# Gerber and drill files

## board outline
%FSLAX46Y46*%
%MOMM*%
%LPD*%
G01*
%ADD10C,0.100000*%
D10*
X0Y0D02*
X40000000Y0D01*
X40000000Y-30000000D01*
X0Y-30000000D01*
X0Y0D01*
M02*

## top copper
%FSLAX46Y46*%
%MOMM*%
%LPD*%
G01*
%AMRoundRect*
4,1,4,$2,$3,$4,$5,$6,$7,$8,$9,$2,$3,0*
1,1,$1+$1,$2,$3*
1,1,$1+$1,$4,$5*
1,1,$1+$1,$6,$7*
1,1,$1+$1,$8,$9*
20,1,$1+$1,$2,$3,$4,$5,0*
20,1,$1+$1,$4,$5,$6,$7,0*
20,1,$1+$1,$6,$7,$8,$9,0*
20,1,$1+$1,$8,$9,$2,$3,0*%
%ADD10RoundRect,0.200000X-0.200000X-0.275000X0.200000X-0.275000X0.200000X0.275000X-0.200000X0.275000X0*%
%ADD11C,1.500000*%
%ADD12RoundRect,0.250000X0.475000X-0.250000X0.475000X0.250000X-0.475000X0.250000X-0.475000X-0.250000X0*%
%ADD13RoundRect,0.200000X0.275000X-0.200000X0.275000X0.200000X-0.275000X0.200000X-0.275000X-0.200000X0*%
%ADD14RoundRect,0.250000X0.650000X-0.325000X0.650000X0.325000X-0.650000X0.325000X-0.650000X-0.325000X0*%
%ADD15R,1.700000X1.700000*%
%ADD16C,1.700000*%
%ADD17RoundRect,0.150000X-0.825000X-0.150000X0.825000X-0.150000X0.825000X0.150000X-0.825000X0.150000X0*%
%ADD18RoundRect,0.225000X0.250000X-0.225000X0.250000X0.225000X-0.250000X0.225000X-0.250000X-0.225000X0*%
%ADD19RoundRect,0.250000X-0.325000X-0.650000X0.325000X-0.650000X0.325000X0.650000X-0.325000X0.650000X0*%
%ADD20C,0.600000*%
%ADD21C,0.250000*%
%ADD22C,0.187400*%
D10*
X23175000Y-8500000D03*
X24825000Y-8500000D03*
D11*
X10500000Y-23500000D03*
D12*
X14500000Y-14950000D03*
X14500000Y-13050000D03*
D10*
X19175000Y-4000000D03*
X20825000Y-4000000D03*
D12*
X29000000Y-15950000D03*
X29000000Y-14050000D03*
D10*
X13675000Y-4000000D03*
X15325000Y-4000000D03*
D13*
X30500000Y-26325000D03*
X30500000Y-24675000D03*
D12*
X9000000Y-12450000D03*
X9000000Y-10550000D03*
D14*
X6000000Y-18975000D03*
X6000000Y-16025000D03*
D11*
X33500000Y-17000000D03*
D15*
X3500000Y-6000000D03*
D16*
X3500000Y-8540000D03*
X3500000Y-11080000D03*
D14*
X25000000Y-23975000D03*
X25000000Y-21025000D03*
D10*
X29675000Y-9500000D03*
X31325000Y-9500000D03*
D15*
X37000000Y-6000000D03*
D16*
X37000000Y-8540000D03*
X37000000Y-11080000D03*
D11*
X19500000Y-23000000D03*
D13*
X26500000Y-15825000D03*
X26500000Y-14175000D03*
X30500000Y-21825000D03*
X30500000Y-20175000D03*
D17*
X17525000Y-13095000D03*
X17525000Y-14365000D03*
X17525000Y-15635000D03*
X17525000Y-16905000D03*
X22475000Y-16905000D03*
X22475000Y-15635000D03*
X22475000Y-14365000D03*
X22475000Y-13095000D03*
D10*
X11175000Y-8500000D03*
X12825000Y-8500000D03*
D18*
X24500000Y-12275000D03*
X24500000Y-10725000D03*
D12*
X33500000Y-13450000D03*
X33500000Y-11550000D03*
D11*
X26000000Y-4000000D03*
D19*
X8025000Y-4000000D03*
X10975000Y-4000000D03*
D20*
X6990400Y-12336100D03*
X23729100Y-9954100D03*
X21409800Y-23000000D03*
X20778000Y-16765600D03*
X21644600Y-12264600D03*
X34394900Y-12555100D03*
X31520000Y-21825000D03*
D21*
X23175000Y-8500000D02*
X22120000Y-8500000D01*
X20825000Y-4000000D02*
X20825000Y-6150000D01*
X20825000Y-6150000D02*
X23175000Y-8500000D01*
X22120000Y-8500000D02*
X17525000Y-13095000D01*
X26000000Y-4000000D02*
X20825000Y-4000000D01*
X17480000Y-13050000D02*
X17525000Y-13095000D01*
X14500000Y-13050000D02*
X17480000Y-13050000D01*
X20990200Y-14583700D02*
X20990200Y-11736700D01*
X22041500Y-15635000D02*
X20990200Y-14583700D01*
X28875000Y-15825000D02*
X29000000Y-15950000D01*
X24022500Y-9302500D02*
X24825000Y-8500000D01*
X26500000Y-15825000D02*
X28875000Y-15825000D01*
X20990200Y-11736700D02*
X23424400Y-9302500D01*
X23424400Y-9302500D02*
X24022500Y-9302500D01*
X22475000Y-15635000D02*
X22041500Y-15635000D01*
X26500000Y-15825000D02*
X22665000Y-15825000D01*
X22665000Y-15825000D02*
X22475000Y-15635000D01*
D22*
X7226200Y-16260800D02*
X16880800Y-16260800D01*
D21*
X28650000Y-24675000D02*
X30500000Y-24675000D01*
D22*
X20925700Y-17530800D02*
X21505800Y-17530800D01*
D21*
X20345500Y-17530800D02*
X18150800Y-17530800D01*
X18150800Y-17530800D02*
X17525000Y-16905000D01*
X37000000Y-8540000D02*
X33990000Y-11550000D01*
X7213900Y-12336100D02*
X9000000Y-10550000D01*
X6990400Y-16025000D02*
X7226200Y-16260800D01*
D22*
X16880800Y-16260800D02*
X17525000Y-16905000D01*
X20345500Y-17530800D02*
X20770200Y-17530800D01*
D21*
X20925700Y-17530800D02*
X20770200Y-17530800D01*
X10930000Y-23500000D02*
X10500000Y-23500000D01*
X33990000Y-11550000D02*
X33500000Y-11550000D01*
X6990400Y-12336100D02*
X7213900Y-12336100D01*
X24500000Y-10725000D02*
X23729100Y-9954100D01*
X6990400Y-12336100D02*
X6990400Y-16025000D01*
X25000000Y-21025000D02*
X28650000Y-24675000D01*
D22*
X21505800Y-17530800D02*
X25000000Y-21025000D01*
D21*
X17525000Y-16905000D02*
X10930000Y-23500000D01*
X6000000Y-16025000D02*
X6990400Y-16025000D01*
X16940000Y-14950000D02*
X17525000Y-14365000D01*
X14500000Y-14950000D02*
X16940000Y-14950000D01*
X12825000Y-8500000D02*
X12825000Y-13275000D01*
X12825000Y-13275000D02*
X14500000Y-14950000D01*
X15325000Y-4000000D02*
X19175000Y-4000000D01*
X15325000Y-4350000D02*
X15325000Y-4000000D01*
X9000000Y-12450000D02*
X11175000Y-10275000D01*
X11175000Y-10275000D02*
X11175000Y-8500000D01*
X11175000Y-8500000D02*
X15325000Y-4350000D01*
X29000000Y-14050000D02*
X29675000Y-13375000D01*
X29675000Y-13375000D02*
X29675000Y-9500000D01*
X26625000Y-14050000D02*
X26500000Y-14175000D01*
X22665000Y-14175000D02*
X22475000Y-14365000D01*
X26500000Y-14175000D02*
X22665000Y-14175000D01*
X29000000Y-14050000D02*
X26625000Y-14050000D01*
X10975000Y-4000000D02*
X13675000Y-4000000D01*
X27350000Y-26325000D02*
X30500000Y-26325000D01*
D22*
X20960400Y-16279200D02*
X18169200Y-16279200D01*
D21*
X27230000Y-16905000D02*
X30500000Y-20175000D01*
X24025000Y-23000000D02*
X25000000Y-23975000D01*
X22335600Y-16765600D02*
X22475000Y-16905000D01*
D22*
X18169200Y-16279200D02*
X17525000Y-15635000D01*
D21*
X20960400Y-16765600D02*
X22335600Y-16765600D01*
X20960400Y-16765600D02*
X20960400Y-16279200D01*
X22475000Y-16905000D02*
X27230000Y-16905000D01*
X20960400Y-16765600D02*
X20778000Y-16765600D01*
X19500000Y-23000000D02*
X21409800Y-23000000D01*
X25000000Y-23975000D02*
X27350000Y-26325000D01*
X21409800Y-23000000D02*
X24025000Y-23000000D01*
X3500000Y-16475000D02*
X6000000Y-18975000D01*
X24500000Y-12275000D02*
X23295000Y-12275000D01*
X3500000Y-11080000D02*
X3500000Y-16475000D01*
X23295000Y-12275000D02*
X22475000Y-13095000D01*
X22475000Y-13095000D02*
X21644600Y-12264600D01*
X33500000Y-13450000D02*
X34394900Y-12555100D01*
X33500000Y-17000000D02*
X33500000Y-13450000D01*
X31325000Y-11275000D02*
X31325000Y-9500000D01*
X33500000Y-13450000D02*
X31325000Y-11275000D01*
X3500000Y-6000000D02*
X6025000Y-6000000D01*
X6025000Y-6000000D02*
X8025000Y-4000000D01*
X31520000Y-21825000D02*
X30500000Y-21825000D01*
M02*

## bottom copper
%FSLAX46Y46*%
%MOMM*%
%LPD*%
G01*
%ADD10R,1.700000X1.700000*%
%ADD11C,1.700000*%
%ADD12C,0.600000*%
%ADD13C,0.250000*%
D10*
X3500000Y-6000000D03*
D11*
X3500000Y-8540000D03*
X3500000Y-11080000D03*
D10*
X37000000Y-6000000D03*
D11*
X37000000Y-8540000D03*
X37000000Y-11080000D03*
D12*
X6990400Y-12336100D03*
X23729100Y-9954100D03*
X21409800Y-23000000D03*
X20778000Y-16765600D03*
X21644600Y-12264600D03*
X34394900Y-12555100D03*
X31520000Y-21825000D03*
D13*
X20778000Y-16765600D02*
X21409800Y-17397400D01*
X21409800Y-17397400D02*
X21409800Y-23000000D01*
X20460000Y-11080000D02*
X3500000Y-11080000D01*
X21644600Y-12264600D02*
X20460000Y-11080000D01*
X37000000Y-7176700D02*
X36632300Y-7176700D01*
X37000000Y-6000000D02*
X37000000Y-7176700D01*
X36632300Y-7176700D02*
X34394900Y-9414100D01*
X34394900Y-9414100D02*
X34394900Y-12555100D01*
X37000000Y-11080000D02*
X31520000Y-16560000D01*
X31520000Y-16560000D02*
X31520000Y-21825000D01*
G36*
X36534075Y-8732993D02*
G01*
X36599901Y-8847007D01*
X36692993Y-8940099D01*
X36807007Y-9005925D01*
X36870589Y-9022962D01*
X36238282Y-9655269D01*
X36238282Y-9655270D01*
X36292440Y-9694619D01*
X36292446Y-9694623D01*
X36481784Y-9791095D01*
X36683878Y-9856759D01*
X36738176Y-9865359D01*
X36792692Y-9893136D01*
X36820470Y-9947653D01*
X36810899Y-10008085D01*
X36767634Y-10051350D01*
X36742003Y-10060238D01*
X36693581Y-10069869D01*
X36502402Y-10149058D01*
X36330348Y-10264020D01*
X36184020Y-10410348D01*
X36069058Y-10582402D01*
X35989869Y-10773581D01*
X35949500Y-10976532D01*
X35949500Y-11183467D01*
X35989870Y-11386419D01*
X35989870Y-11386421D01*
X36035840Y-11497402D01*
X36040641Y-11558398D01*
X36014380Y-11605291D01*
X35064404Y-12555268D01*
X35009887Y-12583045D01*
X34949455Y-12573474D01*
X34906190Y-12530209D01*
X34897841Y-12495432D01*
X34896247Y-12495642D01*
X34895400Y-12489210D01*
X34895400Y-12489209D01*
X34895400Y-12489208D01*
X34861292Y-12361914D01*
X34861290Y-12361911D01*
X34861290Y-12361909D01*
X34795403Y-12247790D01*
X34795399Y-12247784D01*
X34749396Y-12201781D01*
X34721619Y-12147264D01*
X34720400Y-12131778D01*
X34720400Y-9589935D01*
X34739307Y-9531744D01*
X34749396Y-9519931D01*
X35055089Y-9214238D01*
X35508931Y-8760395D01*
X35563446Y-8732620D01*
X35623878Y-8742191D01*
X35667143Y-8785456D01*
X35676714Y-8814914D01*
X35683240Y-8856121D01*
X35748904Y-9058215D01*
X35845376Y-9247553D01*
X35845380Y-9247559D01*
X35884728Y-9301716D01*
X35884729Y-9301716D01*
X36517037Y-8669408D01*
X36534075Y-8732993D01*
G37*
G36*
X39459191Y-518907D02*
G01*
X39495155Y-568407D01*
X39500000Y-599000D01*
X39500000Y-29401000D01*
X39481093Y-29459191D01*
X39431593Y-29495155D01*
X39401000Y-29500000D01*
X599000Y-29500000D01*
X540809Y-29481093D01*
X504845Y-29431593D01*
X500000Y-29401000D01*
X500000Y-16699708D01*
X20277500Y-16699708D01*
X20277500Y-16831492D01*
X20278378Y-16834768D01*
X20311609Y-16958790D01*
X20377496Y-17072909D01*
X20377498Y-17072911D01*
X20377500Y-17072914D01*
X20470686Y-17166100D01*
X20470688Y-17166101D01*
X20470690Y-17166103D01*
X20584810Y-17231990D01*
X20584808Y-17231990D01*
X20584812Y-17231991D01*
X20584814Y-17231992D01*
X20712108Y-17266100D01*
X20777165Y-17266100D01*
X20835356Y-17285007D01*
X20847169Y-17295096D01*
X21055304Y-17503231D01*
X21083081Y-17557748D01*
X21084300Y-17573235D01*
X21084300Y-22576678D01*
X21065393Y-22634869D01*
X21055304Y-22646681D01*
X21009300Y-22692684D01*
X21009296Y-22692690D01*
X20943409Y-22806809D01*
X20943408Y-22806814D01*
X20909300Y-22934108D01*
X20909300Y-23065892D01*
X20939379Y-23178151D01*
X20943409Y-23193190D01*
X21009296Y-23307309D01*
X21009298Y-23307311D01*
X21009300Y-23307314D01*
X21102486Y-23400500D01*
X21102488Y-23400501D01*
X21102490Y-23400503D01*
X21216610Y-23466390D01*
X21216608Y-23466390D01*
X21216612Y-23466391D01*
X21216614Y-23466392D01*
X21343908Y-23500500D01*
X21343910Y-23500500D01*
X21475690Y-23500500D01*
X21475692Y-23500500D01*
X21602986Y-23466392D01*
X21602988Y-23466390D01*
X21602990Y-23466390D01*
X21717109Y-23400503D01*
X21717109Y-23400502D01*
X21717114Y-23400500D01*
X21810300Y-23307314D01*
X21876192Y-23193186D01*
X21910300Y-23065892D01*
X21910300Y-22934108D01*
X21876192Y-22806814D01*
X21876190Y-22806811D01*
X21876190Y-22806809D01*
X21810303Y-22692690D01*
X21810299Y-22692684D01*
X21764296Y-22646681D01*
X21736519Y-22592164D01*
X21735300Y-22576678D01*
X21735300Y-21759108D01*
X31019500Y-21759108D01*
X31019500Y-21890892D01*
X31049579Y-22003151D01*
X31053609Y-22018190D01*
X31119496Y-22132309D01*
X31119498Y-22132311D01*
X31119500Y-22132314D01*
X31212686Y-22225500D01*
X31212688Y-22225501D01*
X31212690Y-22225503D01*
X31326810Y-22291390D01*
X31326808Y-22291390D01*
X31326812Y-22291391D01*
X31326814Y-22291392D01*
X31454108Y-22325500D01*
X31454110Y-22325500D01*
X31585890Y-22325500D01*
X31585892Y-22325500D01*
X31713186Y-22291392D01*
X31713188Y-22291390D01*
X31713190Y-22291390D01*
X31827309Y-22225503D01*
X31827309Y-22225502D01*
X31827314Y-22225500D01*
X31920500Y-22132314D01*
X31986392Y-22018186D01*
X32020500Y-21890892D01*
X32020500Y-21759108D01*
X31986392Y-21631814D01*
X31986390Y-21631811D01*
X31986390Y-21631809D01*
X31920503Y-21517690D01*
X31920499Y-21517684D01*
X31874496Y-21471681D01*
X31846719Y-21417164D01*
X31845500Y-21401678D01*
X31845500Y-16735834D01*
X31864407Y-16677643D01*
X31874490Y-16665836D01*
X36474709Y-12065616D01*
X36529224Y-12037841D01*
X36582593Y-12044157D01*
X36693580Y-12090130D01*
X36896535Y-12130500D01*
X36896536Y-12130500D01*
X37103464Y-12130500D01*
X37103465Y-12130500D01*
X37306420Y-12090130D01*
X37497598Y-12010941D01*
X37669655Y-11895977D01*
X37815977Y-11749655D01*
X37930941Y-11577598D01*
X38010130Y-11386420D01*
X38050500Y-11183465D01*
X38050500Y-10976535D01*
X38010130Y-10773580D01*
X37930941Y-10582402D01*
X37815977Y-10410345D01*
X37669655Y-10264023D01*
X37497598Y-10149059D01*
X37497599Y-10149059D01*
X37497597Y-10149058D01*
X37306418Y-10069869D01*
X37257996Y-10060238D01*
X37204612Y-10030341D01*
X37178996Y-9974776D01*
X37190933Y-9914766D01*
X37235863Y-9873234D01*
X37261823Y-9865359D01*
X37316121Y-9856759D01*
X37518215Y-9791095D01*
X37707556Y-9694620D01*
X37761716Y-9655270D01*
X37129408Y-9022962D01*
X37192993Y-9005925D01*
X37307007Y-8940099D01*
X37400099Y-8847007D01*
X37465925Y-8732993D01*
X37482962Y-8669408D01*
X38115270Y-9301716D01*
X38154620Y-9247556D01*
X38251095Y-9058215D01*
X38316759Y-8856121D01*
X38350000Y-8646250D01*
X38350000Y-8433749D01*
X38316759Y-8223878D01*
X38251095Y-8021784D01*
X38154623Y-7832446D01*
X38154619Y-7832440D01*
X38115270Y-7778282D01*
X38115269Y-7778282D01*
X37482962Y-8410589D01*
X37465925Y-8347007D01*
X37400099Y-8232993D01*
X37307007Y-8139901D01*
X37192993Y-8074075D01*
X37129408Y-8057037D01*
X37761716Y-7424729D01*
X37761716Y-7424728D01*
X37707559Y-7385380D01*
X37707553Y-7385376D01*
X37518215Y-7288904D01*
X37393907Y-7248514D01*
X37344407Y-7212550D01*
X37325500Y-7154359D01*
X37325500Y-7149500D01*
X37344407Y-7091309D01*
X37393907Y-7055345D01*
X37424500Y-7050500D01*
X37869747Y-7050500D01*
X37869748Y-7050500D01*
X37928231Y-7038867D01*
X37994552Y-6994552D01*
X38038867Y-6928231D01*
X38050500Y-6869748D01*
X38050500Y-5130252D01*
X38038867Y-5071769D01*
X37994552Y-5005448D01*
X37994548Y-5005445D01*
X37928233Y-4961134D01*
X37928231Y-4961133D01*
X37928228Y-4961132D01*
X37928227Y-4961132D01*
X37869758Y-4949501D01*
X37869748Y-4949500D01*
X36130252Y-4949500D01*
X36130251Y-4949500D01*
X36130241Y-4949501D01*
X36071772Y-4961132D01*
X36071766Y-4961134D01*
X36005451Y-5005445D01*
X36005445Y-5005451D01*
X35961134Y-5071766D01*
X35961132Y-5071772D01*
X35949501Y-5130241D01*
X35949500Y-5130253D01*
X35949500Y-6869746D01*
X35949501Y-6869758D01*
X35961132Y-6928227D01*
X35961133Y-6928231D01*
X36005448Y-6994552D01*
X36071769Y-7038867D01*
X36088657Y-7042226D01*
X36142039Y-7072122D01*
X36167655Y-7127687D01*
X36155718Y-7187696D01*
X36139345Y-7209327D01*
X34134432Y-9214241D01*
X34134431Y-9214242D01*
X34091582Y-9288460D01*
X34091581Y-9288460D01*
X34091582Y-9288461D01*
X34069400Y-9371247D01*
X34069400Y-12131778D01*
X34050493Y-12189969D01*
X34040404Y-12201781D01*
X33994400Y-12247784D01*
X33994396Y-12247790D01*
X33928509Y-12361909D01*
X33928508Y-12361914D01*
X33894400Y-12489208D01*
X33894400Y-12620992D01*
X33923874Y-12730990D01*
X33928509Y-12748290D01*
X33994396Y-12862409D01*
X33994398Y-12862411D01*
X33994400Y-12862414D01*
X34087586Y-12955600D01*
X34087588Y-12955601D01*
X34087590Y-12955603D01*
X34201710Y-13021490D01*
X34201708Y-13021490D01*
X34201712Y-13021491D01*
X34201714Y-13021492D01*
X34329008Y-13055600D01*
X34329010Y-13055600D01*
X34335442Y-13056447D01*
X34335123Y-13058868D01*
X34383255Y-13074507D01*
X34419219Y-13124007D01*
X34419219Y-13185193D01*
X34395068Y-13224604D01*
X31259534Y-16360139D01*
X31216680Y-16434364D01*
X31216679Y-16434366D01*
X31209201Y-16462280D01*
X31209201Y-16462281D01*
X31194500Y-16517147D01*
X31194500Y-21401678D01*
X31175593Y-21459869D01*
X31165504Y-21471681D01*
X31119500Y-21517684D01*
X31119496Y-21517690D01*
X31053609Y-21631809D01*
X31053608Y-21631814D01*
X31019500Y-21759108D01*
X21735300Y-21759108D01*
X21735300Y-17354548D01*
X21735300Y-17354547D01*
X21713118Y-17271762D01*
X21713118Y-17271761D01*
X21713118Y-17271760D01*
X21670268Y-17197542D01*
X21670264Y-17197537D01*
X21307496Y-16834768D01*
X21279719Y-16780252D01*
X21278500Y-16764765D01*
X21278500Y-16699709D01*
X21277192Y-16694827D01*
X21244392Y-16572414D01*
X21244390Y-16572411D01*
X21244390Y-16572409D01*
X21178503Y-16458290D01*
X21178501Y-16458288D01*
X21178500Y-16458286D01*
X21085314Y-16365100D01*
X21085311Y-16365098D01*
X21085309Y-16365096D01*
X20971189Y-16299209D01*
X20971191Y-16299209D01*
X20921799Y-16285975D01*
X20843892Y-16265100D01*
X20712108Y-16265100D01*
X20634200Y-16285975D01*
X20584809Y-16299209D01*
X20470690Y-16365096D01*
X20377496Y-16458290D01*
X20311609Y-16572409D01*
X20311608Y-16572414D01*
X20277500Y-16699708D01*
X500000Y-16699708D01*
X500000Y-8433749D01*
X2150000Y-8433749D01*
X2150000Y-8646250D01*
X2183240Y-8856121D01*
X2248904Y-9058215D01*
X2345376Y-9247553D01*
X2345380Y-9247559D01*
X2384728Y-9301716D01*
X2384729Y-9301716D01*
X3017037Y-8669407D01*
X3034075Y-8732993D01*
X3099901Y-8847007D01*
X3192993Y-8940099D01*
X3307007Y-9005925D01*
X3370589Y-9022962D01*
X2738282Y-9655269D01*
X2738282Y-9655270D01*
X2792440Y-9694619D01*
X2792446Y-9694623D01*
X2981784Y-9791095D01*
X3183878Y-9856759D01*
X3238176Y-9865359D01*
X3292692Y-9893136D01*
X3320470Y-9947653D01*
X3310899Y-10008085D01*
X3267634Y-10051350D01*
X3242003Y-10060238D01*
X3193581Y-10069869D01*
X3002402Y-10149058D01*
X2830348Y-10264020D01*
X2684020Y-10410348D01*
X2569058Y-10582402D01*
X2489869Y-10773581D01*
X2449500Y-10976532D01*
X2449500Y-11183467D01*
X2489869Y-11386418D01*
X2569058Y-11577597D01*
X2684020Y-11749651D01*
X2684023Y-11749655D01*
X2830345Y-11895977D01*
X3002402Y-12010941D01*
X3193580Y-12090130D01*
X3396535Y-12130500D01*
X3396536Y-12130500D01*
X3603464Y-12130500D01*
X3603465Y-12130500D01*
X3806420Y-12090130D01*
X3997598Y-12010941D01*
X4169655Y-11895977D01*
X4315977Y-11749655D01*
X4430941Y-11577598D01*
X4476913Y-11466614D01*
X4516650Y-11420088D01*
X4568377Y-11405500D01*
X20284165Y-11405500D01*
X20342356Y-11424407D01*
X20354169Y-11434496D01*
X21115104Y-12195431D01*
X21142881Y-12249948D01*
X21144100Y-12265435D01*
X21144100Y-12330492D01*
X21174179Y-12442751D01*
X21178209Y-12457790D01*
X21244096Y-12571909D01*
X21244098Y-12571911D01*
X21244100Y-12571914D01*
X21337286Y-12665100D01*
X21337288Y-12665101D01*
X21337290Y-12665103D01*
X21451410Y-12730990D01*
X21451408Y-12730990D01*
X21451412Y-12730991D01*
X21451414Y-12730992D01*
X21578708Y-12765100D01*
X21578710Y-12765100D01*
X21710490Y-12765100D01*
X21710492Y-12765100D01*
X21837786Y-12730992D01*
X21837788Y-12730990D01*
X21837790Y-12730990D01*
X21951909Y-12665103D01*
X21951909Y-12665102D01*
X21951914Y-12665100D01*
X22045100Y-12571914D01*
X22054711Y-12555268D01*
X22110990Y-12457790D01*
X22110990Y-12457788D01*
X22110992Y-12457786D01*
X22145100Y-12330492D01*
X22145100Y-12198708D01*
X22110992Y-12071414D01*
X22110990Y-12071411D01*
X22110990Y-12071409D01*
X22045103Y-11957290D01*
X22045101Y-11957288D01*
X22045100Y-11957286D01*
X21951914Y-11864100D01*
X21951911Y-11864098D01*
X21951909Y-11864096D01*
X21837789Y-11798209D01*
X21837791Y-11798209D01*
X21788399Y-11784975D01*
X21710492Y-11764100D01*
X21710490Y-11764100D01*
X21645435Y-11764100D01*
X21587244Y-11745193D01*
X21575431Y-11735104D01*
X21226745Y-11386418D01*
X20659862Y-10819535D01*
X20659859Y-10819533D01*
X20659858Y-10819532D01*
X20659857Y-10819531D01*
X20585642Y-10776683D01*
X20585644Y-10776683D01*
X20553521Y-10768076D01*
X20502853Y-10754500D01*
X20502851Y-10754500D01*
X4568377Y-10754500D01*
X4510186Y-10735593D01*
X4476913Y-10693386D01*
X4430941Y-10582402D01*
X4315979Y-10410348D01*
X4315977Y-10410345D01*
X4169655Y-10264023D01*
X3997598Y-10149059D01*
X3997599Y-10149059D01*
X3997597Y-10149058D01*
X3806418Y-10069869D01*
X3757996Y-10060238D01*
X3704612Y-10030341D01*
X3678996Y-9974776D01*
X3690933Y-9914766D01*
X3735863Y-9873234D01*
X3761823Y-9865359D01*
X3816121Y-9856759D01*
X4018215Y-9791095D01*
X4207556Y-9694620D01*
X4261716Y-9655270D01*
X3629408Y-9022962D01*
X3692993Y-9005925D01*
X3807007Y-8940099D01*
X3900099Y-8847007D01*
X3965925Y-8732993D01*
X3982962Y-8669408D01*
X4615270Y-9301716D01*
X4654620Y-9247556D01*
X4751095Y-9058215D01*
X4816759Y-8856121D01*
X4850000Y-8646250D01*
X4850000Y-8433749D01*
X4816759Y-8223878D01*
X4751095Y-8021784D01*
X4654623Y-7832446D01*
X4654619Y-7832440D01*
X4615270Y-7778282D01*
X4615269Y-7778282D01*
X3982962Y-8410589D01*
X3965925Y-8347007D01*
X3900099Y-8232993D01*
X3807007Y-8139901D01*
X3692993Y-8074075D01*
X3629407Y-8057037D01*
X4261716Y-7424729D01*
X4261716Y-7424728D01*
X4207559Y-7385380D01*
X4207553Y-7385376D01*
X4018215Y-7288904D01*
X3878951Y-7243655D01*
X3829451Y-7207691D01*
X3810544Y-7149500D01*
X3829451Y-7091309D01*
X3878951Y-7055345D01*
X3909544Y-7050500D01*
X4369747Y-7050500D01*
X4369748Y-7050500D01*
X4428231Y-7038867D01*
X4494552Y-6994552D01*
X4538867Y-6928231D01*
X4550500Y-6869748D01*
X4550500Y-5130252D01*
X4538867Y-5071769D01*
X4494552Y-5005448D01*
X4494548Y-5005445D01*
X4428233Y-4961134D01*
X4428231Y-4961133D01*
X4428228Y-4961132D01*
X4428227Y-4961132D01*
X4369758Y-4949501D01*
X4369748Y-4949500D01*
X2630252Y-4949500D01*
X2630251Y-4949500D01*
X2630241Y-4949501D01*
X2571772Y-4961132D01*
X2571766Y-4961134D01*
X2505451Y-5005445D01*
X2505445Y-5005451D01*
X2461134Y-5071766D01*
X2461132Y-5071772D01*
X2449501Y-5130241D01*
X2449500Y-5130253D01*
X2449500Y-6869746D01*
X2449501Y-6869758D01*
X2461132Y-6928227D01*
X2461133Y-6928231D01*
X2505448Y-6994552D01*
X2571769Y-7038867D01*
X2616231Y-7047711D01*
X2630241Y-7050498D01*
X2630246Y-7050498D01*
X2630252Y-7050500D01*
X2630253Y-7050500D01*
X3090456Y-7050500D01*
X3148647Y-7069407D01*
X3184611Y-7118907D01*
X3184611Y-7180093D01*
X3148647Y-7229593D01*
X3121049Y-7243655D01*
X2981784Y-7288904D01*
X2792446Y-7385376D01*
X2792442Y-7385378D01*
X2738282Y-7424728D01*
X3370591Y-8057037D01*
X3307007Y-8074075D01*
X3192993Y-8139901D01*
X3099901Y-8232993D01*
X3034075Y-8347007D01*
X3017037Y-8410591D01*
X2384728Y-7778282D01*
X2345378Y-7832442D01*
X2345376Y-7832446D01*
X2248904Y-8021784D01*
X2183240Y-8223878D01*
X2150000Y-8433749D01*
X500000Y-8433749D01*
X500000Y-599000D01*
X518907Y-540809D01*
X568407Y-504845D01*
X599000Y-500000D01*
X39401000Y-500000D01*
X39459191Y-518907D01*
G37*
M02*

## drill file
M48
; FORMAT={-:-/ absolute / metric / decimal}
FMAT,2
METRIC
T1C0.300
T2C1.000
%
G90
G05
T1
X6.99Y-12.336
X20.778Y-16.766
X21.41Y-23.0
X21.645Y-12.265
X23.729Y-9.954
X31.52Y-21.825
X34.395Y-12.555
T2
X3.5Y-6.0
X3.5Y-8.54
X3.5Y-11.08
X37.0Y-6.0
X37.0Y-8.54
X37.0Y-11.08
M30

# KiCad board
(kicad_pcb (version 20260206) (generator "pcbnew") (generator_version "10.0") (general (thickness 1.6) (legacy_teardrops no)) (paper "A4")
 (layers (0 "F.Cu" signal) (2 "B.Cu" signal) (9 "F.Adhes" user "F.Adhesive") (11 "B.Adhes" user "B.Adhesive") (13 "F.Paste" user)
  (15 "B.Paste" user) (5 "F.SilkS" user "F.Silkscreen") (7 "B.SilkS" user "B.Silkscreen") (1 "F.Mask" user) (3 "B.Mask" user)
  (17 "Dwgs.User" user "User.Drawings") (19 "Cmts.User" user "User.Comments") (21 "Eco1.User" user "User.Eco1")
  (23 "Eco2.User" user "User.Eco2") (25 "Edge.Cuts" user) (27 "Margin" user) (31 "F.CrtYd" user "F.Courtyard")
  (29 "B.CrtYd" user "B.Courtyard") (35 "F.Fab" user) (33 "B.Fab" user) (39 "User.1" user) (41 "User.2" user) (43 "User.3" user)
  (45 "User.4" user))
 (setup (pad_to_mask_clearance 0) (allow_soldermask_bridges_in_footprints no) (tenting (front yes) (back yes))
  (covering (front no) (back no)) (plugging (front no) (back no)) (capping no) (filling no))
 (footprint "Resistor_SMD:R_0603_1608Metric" (layer "F.Cu") (at 24 8.5)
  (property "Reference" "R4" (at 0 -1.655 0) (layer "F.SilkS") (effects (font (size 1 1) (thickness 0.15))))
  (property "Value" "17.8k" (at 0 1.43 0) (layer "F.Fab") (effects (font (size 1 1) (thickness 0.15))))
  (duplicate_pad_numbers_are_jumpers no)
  (pad "1" smd roundrect (at -0.825 0) (size 0.8 0.95) (layers "F.Cu" "F.Mask" "F.Paste") (roundrect_rratio 0.25) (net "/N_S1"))
  (pad "2" smd roundrect (at 0.825 0) (size 0.8 0.95) (layers "F.Cu" "F.Mask" "F.Paste") (roundrect_rratio 0.25) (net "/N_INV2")))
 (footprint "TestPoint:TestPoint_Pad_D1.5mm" (layer "F.Cu") (at 10.5 23.5)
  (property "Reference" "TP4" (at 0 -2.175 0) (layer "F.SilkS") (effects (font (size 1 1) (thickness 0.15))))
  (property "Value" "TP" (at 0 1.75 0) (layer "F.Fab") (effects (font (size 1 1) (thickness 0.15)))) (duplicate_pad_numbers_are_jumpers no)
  (pad "1" smd circle (at 0 0) (size 1.5 1.5) (layers "F.Cu" "F.Mask") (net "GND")))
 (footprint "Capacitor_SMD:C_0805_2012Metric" (layer "F.Cu") (at 14.5 14 90)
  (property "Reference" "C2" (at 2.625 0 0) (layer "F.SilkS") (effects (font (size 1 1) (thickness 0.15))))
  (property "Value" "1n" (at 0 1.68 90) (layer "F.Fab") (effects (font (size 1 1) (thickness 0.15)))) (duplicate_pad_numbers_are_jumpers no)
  (pad "1" smd roundrect (at -0.95 0 90) (size 1 1.45) (layers "F.Cu" "F.Mask" "F.Paste") (roundrect_rratio 0.25) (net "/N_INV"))
  (pad "2" smd roundrect (at 0.95 0 90) (size 1 1.45) (layers "F.Cu" "F.Mask" "F.Paste") (roundrect_rratio 0.25) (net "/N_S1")))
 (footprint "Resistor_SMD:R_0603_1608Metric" (layer "F.Cu") (at 20 4)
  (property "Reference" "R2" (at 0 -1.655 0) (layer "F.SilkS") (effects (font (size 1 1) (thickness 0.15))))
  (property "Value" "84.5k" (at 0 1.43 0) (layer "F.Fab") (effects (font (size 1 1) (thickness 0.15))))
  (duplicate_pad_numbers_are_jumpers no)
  (pad "1" smd roundrect (at -0.825 0) (size 0.8 0.95) (layers "F.Cu" "F.Mask" "F.Paste") (roundrect_rratio 0.25) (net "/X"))
  (pad "2" smd roundrect (at 0.825 0) (size 0.8 0.95) (layers "F.Cu" "F.Mask" "F.Paste") (roundrect_rratio 0.25) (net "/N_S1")))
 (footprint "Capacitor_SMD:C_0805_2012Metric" (layer "F.Cu") (at 29 15 90)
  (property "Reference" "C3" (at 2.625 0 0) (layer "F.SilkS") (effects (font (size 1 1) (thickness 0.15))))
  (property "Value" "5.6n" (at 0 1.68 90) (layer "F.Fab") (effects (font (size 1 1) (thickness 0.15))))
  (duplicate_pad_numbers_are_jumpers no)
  (pad "1" smd roundrect (at -0.95 0 90) (size 1 1.45) (layers "F.Cu" "F.Mask" "F.Paste") (roundrect_rratio 0.25) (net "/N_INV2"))
  (pad "2" smd roundrect (at 0.95 0 90) (size 1 1.45) (layers "F.Cu" "F.Mask" "F.Paste") (roundrect_rratio 0.25) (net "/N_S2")))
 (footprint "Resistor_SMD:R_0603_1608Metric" (layer "F.Cu") (at 14.5 4)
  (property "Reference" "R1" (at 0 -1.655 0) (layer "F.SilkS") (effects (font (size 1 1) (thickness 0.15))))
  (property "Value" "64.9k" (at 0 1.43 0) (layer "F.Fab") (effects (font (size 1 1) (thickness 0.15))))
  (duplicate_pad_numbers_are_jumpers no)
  (pad "1" smd roundrect (at -0.825 0) (size 0.8 0.95) (layers "F.Cu" "F.Mask" "F.Paste") (roundrect_rratio 0.25) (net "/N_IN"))
  (pad "2" smd roundrect (at 0.825 0) (size 0.8 0.95) (layers "F.Cu" "F.Mask" "F.Paste") (roundrect_rratio 0.25) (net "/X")))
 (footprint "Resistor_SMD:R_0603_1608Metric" (layer "F.Cu") (at 30.5 25.5 90)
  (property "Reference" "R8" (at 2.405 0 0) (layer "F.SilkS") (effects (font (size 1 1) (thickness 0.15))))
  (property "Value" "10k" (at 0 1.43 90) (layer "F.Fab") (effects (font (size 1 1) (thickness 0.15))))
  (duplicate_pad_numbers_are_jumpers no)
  (pad "1" smd roundrect (at -0.825 0 90) (size 0.8 0.95) (layers "F.Cu" "F.Mask" "F.Paste") (roundrect_rratio 0.25) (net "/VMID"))
  (pad "2" smd roundrect (at 0.825 0 90) (size 0.8 0.95) (layers "F.Cu" "F.Mask" "F.Paste") (roundrect_rratio 0.25) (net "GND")))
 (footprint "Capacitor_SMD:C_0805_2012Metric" (layer "F.Cu") (at 9 11.5 90)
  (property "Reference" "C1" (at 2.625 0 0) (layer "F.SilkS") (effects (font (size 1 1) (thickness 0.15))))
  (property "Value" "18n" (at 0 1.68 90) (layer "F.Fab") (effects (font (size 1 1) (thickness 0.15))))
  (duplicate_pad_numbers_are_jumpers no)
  (pad "1" smd roundrect (at -0.95 0 90) (size 1 1.45) (layers "F.Cu" "F.Mask" "F.Paste") (roundrect_rratio 0.25) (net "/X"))
  (pad "2" smd roundrect (at 0.95 0 90) (size 1 1.45) (layers "F.Cu" "F.Mask" "F.Paste") (roundrect_rratio 0.25) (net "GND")))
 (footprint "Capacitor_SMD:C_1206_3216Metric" (layer "F.Cu") (at 6 17.5 90)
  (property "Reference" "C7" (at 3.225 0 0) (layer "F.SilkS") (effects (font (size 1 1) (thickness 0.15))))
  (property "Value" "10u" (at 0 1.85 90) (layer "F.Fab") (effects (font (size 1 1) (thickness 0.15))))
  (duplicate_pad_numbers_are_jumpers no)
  (pad "1" smd roundrect (at -1.475 0 90) (size 1.15 1.8) (layers "F.Cu" "F.Mask" "F.Paste") (roundrect_rratio 0.217391) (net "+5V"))
  (pad "2" smd roundrect (at 1.475 0 90) (size 1.15 1.8) (layers "F.Cu" "F.Mask" "F.Paste") (roundrect_rratio 0.217391) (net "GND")))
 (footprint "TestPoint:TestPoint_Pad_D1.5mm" (layer "F.Cu") (at 33.5 17)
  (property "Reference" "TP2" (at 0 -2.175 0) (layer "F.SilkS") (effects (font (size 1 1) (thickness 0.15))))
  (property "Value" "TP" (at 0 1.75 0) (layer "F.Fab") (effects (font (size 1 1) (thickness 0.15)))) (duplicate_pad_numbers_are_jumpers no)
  (pad "1" smd circle (at 0 0) (size 1.5 1.5) (layers "F.Cu" "F.Mask") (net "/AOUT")))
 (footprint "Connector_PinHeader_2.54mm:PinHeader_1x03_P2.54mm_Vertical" (layer "F.Cu") (at 3.5 6)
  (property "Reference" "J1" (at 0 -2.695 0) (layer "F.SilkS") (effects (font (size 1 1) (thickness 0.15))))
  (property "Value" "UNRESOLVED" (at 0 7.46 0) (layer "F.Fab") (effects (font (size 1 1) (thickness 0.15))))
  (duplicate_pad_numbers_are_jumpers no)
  (pad "1" thru_hole rect (at 0 0) (size 1.7 1.7) (drill 1) (layers "*.Cu" "*.Mask") (remove_unused_layers no) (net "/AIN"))
  (pad "2" thru_hole circle (at 0 2.54) (size 1.7 1.7) (drill 1) (layers "*.Cu" "*.Mask") (remove_unused_layers no) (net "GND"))
  (pad "3" thru_hole circle (at 0 5.08) (size 1.7 1.7) (drill 1) (layers "*.Cu" "*.Mask") (remove_unused_layers no) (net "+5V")))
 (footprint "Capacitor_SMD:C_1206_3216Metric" (layer "F.Cu") (at 25 22.5 90)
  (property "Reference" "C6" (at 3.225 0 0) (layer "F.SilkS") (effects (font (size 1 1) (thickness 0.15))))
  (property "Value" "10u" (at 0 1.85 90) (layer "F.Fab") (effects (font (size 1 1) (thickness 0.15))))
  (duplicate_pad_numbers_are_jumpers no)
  (pad "1" smd roundrect (at -1.475 0 90) (size 1.15 1.8) (layers "F.Cu" "F.Mask" "F.Paste") (roundrect_rratio 0.217391) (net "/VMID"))
  (pad "2" smd roundrect (at 1.475 0 90) (size 1.15 1.8) (layers "F.Cu" "F.Mask" "F.Paste") (roundrect_rratio 0.217391) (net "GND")))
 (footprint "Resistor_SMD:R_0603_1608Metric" (layer "F.Cu") (at 30.5 9.5)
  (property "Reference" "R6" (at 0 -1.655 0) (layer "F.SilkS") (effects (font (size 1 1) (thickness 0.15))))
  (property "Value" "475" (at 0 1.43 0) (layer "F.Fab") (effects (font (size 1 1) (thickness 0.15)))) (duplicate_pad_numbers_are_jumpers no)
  (pad "1" smd roundrect (at -0.825 0) (size 0.8 0.95) (layers "F.Cu" "F.Mask" "F.Paste") (roundrect_rratio 0.25) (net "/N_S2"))
  (pad "2" smd roundrect (at 0.825 0) (size 0.8 0.95) (layers "F.Cu" "F.Mask" "F.Paste") (roundrect_rratio 0.25) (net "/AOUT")))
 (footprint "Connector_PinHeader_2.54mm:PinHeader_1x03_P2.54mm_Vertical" (layer "F.Cu") (at 37 6)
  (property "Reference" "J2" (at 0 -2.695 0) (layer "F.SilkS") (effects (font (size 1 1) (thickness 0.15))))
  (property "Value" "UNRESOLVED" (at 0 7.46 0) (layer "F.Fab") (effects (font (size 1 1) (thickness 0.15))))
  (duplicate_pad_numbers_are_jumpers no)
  (pad "1" thru_hole rect (at 0 0) (size 1.7 1.7) (drill 1) (layers "*.Cu" "*.Mask") (remove_unused_layers no) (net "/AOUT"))
  (pad "2" thru_hole circle (at 0 2.54) (size 1.7 1.7) (drill 1) (layers "*.Cu" "*.Mask") (remove_unused_layers no) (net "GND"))
  (pad "3" thru_hole circle (at 0 5.08) (size 1.7 1.7) (drill 1) (layers "*.Cu" "*.Mask") (remove_unused_layers no) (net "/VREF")))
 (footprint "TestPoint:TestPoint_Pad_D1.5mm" (layer "F.Cu") (at 19.5 23)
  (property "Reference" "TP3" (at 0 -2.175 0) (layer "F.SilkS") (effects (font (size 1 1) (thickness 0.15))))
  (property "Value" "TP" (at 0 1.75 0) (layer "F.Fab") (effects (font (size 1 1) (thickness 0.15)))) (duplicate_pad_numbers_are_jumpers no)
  (pad "1" smd circle (at 0 0) (size 1.5 1.5) (layers "F.Cu" "F.Mask") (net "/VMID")))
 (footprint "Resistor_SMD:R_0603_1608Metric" (layer "F.Cu") (at 26.5 15 90)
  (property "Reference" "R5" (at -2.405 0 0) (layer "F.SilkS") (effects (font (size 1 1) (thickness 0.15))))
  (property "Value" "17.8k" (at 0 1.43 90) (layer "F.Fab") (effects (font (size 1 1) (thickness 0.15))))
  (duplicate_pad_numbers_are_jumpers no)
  (pad "1" smd roundrect (at -0.825 0 90) (size 0.8 0.95) (layers "F.Cu" "F.Mask" "F.Paste") (roundrect_rratio 0.25) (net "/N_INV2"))
  (pad "2" smd roundrect (at 0.825 0 90) (size 0.8 0.95) (layers "F.Cu" "F.Mask" "F.Paste") (roundrect_rratio 0.25) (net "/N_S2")))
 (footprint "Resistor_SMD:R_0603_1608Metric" (layer "F.Cu") (at 30.5 21 90)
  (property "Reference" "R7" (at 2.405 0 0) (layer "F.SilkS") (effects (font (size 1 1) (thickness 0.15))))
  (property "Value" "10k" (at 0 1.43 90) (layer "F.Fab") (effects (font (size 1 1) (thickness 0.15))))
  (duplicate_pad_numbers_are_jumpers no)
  (pad "1" smd roundrect (at -0.825 0 90) (size 0.8 0.95) (layers "F.Cu" "F.Mask" "F.Paste") (roundrect_rratio 0.25) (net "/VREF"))
  (pad "2" smd roundrect (at 0.825 0 90) (size 0.8 0.95) (layers "F.Cu" "F.Mask" "F.Paste") (roundrect_rratio 0.25) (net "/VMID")))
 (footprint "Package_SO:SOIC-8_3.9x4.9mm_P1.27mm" (layer "F.Cu") (at 20 15)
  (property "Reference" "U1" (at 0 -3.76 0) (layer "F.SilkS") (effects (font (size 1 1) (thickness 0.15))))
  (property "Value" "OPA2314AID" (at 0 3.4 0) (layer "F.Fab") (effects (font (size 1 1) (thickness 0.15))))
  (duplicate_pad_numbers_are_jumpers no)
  (pad "1" smd roundrect (at -2.475 -1.905) (size 1.95 0.6) (layers "F.Cu" "F.Mask" "F.Paste") (roundrect_rratio 0.25) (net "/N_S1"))
  (pad "2" smd roundrect (at -2.475 -0.635) (size 1.95 0.6) (layers "F.Cu" "F.Mask" "F.Paste") (roundrect_rratio 0.25) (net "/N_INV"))
  (pad "3" smd roundrect (at -2.475 0.635) (size 1.95 0.6) (layers "F.Cu" "F.Mask" "F.Paste") (roundrect_rratio 0.25) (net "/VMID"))
  (pad "4" smd roundrect (at -2.475 1.905) (size 1.95 0.6) (layers "F.Cu" "F.Mask" "F.Paste") (roundrect_rratio 0.25) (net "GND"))
  (pad "5" smd roundrect (at 2.475 1.905) (size 1.95 0.6) (layers "F.Cu" "F.Mask" "F.Paste") (roundrect_rratio 0.25) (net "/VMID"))
  (pad "6" smd roundrect (at 2.475 0.635) (size 1.95 0.6) (layers "F.Cu" "F.Mask" "F.Paste") (roundrect_rratio 0.25) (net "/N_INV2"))
  (pad "7" smd roundrect (at 2.475 -0.635) (size 1.95 0.6) (layers "F.Cu" "F.Mask" "F.Paste") (roundrect_rratio 0.25) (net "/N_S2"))
  (pad "8" smd roundrect (at 2.475 -1.905) (size 1.95 0.6) (layers "F.Cu" "F.Mask" "F.Paste") (roundrect_rratio 0.25) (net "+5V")))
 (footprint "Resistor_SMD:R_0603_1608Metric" (layer "F.Cu") (at 12 8.5)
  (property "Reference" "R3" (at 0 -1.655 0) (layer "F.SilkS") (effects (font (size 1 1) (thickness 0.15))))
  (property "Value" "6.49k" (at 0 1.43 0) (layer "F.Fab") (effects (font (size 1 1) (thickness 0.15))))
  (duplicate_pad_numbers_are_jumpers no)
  (pad "1" smd roundrect (at -0.825 0) (size 0.8 0.95) (layers "F.Cu" "F.Mask" "F.Paste") (roundrect_rratio 0.25) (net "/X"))
  (pad "2" smd roundrect (at 0.825 0) (size 0.8 0.95) (layers "F.Cu" "F.Mask" "F.Paste") (roundrect_rratio 0.25) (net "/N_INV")))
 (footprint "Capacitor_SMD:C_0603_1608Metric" (layer "F.Cu") (at 24.5 11.5 90)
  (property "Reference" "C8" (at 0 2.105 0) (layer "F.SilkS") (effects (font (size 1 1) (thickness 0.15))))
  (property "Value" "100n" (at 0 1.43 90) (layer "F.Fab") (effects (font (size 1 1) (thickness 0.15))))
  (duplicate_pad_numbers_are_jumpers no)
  (pad "1" smd roundrect (at -0.775 0 90) (size 0.9 0.95) (layers "F.Cu" "F.Mask" "F.Paste") (roundrect_rratio 0.25) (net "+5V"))
  (pad "2" smd roundrect (at 0.775 0 90) (size 0.9 0.95) (layers "F.Cu" "F.Mask" "F.Paste") (roundrect_rratio 0.25) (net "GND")))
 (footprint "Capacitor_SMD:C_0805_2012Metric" (layer "F.Cu") (at 33.5 12.5 90)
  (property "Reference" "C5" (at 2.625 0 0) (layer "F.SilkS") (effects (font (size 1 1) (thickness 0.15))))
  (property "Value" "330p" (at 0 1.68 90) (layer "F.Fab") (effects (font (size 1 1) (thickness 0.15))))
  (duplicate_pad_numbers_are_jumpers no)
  (pad "1" smd roundrect (at -0.95 0 90) (size 1 1.45) (layers "F.Cu" "F.Mask" "F.Paste") (roundrect_rratio 0.25) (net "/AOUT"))
  (pad "2" smd roundrect (at 0.95 0 90) (size 1 1.45) (layers "F.Cu" "F.Mask" "F.Paste") (roundrect_rratio 0.25) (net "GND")))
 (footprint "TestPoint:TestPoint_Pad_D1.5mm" (layer "F.Cu") (at 26 4)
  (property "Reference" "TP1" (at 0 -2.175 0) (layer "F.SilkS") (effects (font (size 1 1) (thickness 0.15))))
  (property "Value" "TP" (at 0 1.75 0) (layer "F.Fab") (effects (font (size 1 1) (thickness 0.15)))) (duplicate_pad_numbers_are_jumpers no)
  (pad "1" smd circle (at 0 0) (size 1.5 1.5) (layers "F.Cu" "F.Mask") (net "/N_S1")))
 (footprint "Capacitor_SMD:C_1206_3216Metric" (layer "F.Cu") (at 9.5 4)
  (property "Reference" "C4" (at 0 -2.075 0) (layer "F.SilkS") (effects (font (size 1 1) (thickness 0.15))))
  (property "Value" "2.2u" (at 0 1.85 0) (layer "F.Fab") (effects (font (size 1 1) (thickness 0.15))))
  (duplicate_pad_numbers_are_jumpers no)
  (pad "1" smd roundrect (at -1.475 0) (size 1.15 1.8) (layers "F.Cu" "F.Mask" "F.Paste") (roundrect_rratio 0.217391) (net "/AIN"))
  (pad "2" smd roundrect (at 1.475 0) (size 1.15 1.8) (layers "F.Cu" "F.Mask" "F.Paste") (roundrect_rratio 0.217391) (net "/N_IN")))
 (gr_rect (start 0 0) (end 40 30) (stroke (width 0.1) (type default)) (fill no) (layer "Edge.Cuts"))
 (segment (start 23.175 8.5) (end 22.12 8.5) (width 0.25) (layer "F.Cu") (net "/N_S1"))
 (segment (start 20.825 4) (end 20.825 6.15) (width 0.25) (layer "F.Cu") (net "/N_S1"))
 (segment (start 20.825 6.15) (end 23.175 8.5) (width 0.25) (layer "F.Cu") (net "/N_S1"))
 (segment (start 22.12 8.5) (end 17.525 13.095) (width 0.25) (layer "F.Cu") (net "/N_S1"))
 (segment (start 26 4) (end 20.825 4) (width 0.25) (layer "F.Cu") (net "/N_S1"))
 (segment (start 17.48 13.05) (end 17.525 13.095) (width 0.25) (layer "F.Cu") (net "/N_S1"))
 (segment (start 14.5 13.05) (end 17.48 13.05) (width 0.25) (layer "F.Cu") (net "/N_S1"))
 (segment (start 20.9902 14.5837) (end 20.9902 11.7367) (width 0.25) (layer "F.Cu") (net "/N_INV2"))
 (segment (start 22.0415 15.635) (end 20.9902 14.5837) (width 0.25) (layer "F.Cu") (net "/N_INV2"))
 (segment (start 28.875 15.825) (end 29 15.95) (width 0.25) (layer "F.Cu") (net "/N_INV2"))
 (segment (start 24.0225 9.3025) (end 24.825 8.5) (width 0.25) (layer "F.Cu") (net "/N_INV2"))
 (segment (start 26.5 15.825) (end 28.875 15.825) (width 0.25) (layer "F.Cu") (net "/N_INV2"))
 (segment (start 20.9902 11.7367) (end 23.4244 9.3025) (width 0.25) (layer "F.Cu") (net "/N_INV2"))
 (segment (start 23.4244 9.3025) (end 24.0225 9.3025) (width 0.25) (layer "F.Cu") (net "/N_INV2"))
 (segment (start 22.475 15.635) (end 22.0415 15.635) (width 0.25) (layer "F.Cu") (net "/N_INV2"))
 (segment (start 26.5 15.825) (end 22.665 15.825) (width 0.25) (layer "F.Cu") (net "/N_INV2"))
 (segment (start 22.665 15.825) (end 22.475 15.635) (width 0.25) (layer "F.Cu") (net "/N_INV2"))
 (segment (start 7.2262 16.2608) (end 16.8808 16.2608) (width 0.1874) (layer "F.Cu") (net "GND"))
 (segment (start 28.65 24.675) (end 30.5 24.675) (width 0.25) (layer "F.Cu") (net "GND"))
 (segment (start 20.9257 17.5308) (end 21.5058 17.5308) (width 0.1874) (layer "F.Cu") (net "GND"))
 (segment (start 20.3455 17.5308) (end 18.1508 17.5308) (width 0.25) (layer "F.Cu") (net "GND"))
 (segment (start 18.1508 17.5308) (end 17.525 16.905) (width 0.25) (layer "F.Cu") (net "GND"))
 (segment (start 37 8.54) (end 33.99 11.55) (width 0.25) (layer "F.Cu") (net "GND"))
 (segment (start 7.2139 12.3361) (end 9 10.55) (width 0.25) (layer "F.Cu") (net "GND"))
 (segment (start 6.9904 16.025) (end 7.2262 16.2608) (width 0.25) (layer "F.Cu") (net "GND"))
 (segment (start 16.8808 16.2608) (end 17.525 16.905) (width 0.1874) (layer "F.Cu") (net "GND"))
 (segment (start 20.3455 17.5308) (end 20.7702 17.5308) (width 0.1874) (layer "F.Cu") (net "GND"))
 (segment (start 20.9257 17.5308) (end 20.7702 17.5308) (width 0.25) (layer "F.Cu") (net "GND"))
 (segment (start 10.93 23.5) (end 10.5 23.5) (width 0.25) (layer "F.Cu") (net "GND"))
 (segment (start 33.99 11.55) (end 33.5 11.55) (width 0.25) (layer "F.Cu") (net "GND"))
 (segment (start 6.9904 12.3361) (end 7.2139 12.3361) (width 0.25) (layer "F.Cu") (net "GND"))
 (segment (start 24.5 10.725) (end 23.7291 9.9541) (width 0.25) (layer "F.Cu") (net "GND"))
 (segment (start 6.9904 12.3361) (end 6.9904 16.025) (width 0.25) (layer "F.Cu") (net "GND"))
 (segment (start 25 21.025) (end 28.65 24.675) (width 0.25) (layer "F.Cu") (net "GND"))
 (segment (start 21.5058 17.5308) (end 25 21.025) (width 0.1874) (layer "F.Cu") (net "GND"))
 (segment (start 17.525 16.905) (end 10.93 23.5) (width 0.25) (layer "F.Cu") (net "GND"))
 (segment (start 6 16.025) (end 6.9904 16.025) (width 0.25) (layer "F.Cu") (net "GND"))
 (via (at 6.9904 12.3361) (size 0.6) (drill 0.3) (layers "F.Cu" "B.Cu") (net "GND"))
 (via (at 23.7291 9.9541) (size 0.6) (drill 0.3) (layers "F.Cu" "B.Cu") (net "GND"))
 (segment (start 16.94 14.95) (end 17.525 14.365) (width 0.25) (layer "F.Cu") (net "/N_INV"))
 (segment (start 14.5 14.95) (end 16.94 14.95) (width 0.25) (layer "F.Cu") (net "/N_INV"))
 (segment (start 12.825 8.5) (end 12.825 13.275) (width 0.25) (layer "F.Cu") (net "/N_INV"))
 (segment (start 12.825 13.275) (end 14.5 14.95) (width 0.25) (layer "F.Cu") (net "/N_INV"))
 (segment (start 15.325 4) (end 19.175 4) (width 0.25) (layer "F.Cu") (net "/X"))
 (segment (start 15.325 4.35) (end 15.325 4) (width 0.25) (layer "F.Cu") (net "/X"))
 (segment (start 9 12.45) (end 11.175 10.275) (width 0.25) (layer "F.Cu") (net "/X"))
 (segment (start 11.175 10.275) (end 11.175 8.5) (width 0.25) (layer "F.Cu") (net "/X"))
 (segment (start 11.175 8.5) (end 15.325 4.35) (width 0.25) (layer "F.Cu") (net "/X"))
 (segment (start 29 14.05) (end 29.675 13.375) (width 0.25) (layer "F.Cu") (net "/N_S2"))
 (segment (start 29.675 13.375) (end 29.675 9.5) (width 0.25) (layer "F.Cu") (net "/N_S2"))
 (segment (start 26.625 14.05) (end 26.5 14.175) (width 0.25) (layer "F.Cu") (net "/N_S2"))
 (segment (start 22.665 14.175) (end 22.475 14.365) (width 0.25) (layer "F.Cu") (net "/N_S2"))
 (segment (start 26.5 14.175) (end 22.665 14.175) (width 0.25) (layer "F.Cu") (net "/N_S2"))
 (segment (start 29 14.05) (end 26.625 14.05) (width 0.25) (layer "F.Cu") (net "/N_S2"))
 (segment (start 10.975 4) (end 13.675 4) (width 0.25) (layer "F.Cu") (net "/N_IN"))
 (segment (start 27.35 26.325) (end 30.5 26.325) (width 0.25) (layer "F.Cu") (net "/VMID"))
 (segment (start 20.9604 16.2792) (end 18.1692 16.2792) (width 0.1874) (layer "F.Cu") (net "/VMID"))
 (segment (start 27.23 16.905) (end 30.5 20.175) (width 0.25) (layer "F.Cu") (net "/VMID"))
 (segment (start 24.025 23) (end 25 23.975) (width 0.25) (layer "F.Cu") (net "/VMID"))
 (segment (start 22.3356 16.7656) (end 22.475 16.905) (width 0.25) (layer "F.Cu") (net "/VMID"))
 (segment (start 18.1692 16.2792) (end 17.525 15.635) (width 0.1874) (layer "F.Cu") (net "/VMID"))
 (segment (start 20.9604 16.7656) (end 22.3356 16.7656) (width 0.25) (layer "F.Cu") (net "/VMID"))
 (segment (start 20.9604 16.7656) (end 20.9604 16.2792) (width 0.25) (layer "F.Cu") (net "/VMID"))
 (segment (start 22.475 16.905) (end 27.23 16.905) (width 0.25) (layer "F.Cu") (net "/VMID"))
 (segment (start 20.9604 16.7656) (end 20.778 16.7656) (width 0.25) (layer "F.Cu") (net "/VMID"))
 (segment (start 19.5 23) (end 21.4098 23) (width 0.25) (layer "F.Cu") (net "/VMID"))
 (segment (start 25 23.975) (end 27.35 26.325) (width 0.25) (layer "F.Cu") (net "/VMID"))
 (segment (start 21.4098 23) (end 24.025 23) (width 0.25) (layer "F.Cu") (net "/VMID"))
 (via (at 21.4098 23) (size 0.6) (drill 0.3) (layers "F.Cu" "B.Cu") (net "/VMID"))
 (via (at 20.778 16.7656) (size 0.6) (drill 0.3) (layers "F.Cu" "B.Cu") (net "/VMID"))
 (segment (start 20.778 16.7656) (end 21.4098 17.3974) (width 0.25) (layer "B.Cu") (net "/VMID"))
 (segment (start 21.4098 17.3974) (end 21.4098 23) (width 0.25) (layer "B.Cu") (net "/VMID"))
 (segment (start 3.5 16.475) (end 6 18.975) (width 0.25) (layer "F.Cu") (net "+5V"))
 (segment (start 24.5 12.275) (end 23.295 12.275) (width 0.25) (layer "F.Cu") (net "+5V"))
 (segment (start 3.5 11.08) (end 3.5 16.475) (width 0.25) (layer "F.Cu") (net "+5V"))
 (segment (start 23.295 12.275) (end 22.475 13.095) (width 0.25) (layer "F.Cu") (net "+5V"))
 (segment (start 22.475 13.095) (end 21.6446 12.2646) (width 0.25) (layer "F.Cu") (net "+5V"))
 (via (at 21.6446 12.2646) (size 0.6) (drill 0.3) (layers "F.Cu" "B.Cu") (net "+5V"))
 (segment (start 20.46 11.08) (end 3.5 11.08) (width 0.25) (layer "B.Cu") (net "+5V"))
 (segment (start 21.6446 12.2646) (end 20.46 11.08) (width 0.25) (layer "B.Cu") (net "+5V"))
 (segment (start 33.5 13.45) (end 34.3949 12.5551) (width 0.25) (layer "F.Cu") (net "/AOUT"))
 (segment (start 33.5 17) (end 33.5 13.45) (width 0.25) (layer "F.Cu") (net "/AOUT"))
 (segment (start 31.325 11.275) (end 31.325 9.5) (width 0.25) (layer "F.Cu") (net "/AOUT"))
 (segment (start 33.5 13.45) (end 31.325 11.275) (width 0.25) (layer "F.Cu") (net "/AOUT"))
 (via (at 34.3949 12.5551) (size 0.6) (drill 0.3) (layers "F.Cu" "B.Cu") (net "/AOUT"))
 (segment (start 37 7.1767) (end 36.6323 7.1767) (width 0.25) (layer "B.Cu") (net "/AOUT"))
 (segment (start 37 6) (end 37 7.1767) (width 0.25) (layer "B.Cu") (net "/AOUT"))
 (segment (start 36.6323 7.1767) (end 34.3949 9.4141) (width 0.25) (layer "B.Cu") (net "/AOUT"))
 (segment (start 34.3949 9.4141) (end 34.3949 12.5551) (width 0.25) (layer "B.Cu") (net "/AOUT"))
 (segment (start 3.5 6) (end 6.025 6) (width 0.25) (layer "F.Cu") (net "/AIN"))
 (segment (start 6.025 6) (end 8.025 4) (width 0.25) (layer "F.Cu") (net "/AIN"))
 (segment (start 31.52 21.825) (end 30.5 21.825) (width 0.25) (layer "F.Cu") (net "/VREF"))
 (via (at 31.52 21.825) (size 0.6) (drill 0.3) (layers "F.Cu" "B.Cu") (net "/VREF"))
 (segment (start 37 11.08) (end 31.52 16.56) (width 0.25) (layer "B.Cu") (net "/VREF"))
 (segment (start 31.52 16.56) (end 31.52 21.825) (width 0.25) (layer "B.Cu") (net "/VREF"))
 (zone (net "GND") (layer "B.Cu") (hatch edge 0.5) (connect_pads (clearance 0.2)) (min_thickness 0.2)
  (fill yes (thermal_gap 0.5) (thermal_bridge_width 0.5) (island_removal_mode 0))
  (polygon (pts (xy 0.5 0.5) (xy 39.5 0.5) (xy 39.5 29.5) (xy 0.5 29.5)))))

